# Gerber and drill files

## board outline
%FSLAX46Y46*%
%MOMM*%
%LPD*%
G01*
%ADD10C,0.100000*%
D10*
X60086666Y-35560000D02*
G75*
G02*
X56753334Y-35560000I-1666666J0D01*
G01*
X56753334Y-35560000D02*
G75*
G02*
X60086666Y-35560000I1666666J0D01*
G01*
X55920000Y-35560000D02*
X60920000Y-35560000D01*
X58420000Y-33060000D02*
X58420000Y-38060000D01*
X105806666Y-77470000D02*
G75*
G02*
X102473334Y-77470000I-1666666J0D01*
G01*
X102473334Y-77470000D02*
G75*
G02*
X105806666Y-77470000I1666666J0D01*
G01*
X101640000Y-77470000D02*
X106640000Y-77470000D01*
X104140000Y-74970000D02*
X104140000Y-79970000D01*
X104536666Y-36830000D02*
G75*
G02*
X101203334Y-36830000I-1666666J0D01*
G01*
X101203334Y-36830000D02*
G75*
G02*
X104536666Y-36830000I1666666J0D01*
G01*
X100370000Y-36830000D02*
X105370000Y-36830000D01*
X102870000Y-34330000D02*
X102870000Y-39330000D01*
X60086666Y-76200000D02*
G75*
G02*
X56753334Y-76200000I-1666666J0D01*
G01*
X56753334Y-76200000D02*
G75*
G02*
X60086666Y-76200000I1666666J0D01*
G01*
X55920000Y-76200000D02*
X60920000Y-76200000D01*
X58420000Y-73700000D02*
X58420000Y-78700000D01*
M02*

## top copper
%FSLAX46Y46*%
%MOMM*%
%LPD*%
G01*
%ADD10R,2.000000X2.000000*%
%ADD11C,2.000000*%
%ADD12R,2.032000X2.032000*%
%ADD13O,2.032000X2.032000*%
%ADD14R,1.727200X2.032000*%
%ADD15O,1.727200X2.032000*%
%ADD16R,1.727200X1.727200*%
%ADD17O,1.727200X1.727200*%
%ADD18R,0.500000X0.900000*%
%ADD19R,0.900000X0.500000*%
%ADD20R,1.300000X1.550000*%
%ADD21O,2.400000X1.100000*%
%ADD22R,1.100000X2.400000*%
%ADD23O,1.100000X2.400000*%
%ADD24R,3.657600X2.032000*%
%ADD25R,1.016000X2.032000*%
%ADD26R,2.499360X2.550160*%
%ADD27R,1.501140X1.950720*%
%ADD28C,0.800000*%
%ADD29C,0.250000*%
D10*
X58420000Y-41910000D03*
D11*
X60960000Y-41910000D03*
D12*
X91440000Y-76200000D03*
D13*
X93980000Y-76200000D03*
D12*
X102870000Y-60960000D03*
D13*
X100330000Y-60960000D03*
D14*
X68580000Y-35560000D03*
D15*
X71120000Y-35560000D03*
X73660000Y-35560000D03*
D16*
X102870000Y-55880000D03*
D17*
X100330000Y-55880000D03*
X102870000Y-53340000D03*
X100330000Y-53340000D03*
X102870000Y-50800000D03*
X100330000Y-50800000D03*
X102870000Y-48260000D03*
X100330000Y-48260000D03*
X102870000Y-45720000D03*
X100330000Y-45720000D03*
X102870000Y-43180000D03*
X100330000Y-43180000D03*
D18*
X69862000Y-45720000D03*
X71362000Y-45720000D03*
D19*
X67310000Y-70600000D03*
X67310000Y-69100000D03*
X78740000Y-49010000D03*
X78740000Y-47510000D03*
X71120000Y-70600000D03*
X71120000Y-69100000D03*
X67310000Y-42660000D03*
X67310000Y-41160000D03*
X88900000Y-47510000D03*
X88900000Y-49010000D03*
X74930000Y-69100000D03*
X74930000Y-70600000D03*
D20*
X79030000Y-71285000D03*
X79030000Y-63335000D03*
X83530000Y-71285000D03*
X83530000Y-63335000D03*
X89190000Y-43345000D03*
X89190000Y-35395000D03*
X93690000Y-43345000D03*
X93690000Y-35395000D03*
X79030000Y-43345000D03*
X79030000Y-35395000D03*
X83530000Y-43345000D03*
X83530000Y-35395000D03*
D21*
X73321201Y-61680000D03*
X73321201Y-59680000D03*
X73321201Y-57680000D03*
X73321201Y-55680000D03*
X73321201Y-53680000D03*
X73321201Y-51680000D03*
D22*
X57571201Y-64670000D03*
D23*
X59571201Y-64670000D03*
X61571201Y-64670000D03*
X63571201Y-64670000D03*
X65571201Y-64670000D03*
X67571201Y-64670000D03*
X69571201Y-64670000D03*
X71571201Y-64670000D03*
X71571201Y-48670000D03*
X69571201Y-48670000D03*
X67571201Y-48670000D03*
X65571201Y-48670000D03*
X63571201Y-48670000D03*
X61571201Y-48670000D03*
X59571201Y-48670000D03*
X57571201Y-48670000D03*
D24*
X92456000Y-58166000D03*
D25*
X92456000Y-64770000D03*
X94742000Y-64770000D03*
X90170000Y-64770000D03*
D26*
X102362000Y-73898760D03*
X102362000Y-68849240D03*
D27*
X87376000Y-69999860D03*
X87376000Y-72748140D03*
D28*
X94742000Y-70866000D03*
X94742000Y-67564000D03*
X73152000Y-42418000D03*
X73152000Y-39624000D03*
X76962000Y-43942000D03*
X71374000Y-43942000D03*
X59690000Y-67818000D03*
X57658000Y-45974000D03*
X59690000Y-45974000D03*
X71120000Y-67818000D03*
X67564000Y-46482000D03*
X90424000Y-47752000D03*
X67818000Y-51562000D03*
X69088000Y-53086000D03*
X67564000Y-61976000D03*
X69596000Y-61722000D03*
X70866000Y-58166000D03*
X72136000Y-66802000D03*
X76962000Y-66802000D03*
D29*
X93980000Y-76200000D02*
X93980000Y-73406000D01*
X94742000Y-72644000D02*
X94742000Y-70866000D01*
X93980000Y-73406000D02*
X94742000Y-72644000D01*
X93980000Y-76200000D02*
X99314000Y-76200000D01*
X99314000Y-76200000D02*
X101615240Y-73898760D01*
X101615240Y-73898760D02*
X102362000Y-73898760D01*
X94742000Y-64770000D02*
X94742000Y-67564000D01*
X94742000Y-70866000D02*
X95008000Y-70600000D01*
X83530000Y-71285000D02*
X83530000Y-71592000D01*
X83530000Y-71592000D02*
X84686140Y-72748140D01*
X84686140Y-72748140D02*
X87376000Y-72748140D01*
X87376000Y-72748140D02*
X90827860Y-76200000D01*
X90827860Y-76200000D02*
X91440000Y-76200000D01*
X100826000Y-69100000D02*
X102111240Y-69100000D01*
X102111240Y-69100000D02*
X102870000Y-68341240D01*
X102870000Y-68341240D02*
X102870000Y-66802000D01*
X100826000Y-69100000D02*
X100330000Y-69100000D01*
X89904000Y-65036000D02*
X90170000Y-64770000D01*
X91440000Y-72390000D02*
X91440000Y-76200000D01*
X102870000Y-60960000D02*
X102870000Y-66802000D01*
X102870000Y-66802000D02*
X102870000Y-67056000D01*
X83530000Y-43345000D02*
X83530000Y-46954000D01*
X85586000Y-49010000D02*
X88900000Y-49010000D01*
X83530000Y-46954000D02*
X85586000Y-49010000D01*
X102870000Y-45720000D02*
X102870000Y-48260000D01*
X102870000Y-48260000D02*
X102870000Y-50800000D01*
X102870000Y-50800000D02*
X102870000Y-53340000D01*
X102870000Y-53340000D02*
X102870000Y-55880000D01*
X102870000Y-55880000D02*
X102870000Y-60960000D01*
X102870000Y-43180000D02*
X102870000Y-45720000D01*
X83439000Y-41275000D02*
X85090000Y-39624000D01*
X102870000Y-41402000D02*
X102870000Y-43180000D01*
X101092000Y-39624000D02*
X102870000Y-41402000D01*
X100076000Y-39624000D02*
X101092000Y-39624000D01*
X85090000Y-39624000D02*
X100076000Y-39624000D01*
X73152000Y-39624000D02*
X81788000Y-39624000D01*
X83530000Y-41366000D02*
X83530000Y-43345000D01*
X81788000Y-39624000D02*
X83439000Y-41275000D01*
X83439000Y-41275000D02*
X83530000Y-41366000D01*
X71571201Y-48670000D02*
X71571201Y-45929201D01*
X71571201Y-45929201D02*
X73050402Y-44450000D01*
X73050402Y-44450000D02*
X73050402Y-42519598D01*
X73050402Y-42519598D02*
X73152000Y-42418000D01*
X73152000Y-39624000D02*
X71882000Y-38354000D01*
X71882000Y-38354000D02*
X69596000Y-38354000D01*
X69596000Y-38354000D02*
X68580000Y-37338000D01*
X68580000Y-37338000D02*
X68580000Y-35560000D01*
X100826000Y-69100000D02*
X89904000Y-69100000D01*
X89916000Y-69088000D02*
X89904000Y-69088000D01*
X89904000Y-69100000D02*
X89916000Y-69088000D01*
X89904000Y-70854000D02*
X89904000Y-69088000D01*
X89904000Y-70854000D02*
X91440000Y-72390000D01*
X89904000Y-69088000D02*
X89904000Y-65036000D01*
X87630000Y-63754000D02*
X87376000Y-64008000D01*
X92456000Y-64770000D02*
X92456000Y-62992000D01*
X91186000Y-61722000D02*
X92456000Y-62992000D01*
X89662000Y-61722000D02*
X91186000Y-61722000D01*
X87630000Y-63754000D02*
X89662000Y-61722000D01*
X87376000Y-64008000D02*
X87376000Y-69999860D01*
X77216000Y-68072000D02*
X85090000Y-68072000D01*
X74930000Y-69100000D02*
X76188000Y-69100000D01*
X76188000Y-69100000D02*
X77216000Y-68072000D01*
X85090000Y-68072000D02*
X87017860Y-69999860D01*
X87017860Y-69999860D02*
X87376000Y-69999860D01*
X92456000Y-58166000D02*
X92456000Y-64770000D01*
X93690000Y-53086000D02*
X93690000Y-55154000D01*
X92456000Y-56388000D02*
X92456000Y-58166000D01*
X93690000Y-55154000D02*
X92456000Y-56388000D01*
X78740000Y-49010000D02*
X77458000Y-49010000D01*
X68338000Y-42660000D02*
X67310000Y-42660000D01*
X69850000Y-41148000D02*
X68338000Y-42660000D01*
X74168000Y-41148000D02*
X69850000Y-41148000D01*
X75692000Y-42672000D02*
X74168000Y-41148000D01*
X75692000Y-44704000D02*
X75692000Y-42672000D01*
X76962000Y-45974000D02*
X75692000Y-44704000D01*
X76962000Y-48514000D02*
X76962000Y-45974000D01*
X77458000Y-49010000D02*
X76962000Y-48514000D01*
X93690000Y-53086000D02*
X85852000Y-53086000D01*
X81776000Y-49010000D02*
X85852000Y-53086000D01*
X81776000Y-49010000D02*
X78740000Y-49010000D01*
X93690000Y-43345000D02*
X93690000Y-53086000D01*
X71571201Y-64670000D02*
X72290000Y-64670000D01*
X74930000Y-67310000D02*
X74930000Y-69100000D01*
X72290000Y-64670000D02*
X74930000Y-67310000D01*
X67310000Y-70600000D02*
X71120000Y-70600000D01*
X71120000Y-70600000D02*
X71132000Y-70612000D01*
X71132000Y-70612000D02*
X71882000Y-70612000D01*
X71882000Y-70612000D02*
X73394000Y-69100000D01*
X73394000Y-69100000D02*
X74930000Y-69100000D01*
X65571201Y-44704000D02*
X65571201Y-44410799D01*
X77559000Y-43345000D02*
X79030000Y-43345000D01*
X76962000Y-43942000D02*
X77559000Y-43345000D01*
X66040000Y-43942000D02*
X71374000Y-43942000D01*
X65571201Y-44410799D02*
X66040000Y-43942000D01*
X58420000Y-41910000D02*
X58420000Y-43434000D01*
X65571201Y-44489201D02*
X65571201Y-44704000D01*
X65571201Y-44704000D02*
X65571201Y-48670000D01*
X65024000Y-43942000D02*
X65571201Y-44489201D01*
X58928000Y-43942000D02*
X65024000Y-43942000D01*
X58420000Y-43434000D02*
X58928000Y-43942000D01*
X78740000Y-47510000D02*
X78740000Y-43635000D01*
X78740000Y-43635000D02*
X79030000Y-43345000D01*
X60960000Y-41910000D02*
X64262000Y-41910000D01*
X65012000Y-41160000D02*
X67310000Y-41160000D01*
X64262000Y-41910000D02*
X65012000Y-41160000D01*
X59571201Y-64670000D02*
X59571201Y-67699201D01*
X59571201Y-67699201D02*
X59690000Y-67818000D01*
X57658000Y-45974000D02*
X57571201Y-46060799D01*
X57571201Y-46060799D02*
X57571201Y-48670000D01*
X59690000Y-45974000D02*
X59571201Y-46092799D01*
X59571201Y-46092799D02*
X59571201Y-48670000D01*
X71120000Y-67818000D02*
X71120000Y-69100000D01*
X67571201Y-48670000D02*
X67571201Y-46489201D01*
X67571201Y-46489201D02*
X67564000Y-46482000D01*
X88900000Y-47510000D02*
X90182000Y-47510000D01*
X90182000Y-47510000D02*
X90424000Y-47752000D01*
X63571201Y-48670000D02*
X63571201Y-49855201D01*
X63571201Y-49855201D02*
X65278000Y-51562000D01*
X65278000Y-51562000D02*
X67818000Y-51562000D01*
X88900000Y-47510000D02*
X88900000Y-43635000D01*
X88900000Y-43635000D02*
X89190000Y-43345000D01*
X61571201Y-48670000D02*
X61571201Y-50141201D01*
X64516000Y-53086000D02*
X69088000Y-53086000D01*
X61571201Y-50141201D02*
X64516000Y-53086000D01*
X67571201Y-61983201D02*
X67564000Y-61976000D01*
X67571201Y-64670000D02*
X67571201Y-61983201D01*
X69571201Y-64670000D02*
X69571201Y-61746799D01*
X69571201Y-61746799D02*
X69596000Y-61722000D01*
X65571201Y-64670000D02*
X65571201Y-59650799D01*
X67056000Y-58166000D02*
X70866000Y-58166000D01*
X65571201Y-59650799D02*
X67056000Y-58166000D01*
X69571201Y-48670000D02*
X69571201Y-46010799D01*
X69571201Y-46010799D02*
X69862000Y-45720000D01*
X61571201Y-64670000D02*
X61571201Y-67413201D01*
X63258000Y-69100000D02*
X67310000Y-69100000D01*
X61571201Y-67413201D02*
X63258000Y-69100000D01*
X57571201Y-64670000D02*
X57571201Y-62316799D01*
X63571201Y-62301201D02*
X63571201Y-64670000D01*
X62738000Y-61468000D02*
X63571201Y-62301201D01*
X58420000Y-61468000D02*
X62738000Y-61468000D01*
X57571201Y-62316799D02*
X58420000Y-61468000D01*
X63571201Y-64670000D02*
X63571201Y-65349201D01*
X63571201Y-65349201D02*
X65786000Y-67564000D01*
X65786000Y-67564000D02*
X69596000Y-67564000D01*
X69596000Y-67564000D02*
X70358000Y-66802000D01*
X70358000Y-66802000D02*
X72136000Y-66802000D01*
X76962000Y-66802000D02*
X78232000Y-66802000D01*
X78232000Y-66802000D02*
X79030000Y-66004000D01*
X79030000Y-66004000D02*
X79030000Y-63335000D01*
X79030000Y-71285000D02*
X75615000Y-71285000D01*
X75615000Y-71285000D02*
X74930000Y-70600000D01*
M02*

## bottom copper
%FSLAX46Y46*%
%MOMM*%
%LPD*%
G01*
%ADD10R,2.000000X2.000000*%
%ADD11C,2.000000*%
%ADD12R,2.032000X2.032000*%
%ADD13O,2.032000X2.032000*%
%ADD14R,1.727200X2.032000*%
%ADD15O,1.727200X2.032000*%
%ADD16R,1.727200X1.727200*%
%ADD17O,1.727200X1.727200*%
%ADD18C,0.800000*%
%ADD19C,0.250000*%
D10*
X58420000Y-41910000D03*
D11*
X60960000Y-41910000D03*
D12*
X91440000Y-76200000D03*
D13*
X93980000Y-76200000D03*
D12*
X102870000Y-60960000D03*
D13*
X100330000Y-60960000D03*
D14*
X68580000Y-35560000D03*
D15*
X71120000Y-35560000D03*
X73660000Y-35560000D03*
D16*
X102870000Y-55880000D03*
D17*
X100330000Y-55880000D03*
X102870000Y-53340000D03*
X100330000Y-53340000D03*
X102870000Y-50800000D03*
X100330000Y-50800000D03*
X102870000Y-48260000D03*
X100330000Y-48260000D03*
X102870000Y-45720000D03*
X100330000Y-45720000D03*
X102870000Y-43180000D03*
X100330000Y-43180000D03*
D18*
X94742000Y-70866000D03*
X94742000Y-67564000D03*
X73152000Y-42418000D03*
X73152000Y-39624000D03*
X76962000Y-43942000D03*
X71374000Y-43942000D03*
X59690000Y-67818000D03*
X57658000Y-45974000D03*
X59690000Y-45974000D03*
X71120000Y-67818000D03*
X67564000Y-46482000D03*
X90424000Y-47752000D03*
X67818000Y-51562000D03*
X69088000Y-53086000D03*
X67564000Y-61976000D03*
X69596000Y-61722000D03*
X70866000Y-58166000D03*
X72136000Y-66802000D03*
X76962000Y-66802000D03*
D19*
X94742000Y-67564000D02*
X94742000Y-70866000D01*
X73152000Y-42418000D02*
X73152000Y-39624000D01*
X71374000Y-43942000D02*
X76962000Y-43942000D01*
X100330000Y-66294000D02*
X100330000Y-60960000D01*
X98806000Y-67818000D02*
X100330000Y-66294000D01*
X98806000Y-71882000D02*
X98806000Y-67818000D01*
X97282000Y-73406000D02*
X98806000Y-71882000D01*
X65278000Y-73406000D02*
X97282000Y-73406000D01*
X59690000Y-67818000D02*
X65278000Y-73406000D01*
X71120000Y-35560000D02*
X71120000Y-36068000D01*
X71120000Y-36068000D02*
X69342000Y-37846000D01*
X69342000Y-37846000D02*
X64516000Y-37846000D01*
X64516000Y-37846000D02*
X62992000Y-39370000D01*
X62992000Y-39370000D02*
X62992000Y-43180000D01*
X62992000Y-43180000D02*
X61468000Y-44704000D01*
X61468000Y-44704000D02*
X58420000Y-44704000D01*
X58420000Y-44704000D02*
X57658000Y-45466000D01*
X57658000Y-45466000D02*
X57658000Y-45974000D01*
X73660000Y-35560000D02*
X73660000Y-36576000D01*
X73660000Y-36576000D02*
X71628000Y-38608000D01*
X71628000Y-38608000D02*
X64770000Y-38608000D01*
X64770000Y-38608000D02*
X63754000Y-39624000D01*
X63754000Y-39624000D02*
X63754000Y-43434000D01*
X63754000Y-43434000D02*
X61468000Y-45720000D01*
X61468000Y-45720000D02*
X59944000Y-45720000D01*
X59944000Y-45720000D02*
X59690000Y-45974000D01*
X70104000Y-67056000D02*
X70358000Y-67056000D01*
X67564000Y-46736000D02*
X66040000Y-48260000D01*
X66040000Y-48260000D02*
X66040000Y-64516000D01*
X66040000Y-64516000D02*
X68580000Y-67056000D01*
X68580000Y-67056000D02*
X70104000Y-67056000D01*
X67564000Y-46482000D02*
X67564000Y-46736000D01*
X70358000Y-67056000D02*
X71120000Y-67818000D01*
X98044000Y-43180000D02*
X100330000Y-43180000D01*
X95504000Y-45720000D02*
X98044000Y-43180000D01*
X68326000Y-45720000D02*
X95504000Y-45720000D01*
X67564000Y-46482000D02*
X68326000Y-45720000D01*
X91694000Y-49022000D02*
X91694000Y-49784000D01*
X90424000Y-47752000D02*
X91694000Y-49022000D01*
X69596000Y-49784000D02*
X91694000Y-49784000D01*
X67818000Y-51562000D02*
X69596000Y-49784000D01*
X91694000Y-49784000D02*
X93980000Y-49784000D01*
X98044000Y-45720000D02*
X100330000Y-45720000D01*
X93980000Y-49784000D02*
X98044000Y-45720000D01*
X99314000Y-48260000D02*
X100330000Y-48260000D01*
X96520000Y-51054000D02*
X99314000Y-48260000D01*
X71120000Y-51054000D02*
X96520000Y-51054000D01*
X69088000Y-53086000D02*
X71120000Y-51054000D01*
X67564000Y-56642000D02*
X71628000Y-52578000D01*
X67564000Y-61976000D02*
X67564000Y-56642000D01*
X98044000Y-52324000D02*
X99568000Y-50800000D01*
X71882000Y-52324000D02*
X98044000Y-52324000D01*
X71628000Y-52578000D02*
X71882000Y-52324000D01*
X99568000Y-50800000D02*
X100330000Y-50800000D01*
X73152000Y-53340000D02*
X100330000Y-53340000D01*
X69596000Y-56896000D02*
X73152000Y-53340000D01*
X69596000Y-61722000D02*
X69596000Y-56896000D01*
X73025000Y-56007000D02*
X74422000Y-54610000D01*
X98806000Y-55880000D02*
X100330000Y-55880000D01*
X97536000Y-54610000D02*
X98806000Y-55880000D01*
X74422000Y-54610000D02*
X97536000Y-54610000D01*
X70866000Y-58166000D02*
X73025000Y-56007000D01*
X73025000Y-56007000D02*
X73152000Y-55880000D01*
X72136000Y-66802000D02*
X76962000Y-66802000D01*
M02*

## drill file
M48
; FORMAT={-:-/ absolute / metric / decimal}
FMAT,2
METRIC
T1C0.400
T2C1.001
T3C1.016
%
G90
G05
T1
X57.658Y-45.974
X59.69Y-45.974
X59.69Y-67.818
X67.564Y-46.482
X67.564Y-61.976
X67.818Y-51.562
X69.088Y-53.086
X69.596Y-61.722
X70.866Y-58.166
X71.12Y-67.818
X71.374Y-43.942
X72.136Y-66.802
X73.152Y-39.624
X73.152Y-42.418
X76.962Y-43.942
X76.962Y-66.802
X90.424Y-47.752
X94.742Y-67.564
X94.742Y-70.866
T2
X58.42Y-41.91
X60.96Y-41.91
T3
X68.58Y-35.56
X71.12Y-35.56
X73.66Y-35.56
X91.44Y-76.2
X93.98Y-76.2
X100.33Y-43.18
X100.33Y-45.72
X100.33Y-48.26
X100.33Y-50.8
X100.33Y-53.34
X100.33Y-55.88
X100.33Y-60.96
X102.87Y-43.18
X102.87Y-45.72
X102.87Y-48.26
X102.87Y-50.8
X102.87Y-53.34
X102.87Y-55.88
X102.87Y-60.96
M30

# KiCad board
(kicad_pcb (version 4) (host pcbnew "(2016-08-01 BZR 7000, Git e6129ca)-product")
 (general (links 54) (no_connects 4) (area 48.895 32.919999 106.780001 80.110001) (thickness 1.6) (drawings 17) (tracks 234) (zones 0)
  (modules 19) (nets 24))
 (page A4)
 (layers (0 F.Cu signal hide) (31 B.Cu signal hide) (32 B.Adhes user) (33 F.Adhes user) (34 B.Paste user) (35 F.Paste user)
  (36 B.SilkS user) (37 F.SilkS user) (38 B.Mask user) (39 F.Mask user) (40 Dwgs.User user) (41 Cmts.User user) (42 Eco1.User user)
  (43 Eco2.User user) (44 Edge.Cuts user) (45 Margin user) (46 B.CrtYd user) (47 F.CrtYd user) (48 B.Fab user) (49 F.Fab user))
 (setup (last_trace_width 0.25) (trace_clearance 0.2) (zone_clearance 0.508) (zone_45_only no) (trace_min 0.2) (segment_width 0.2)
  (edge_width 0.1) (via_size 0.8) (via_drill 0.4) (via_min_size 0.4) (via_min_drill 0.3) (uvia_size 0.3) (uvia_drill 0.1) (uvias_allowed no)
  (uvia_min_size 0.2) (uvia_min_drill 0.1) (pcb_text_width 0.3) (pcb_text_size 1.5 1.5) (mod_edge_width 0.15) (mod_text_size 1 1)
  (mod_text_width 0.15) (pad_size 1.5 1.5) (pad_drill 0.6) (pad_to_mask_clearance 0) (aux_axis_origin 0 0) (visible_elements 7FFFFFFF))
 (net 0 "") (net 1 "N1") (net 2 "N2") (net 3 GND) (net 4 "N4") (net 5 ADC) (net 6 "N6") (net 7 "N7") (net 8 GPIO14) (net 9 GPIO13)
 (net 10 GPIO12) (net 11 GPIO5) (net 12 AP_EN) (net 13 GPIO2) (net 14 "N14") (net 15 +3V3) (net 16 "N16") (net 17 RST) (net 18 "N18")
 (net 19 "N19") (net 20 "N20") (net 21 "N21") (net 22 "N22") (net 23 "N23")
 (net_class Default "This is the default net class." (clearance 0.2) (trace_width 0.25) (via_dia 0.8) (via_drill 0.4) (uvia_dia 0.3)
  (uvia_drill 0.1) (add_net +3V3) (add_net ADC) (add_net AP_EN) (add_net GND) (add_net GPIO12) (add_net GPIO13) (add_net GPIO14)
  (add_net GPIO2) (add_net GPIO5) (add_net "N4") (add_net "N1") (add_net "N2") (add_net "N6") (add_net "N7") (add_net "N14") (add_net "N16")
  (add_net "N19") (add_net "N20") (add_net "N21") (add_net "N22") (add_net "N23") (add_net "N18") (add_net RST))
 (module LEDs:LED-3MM (layer F.Cu) (at 58.42 41.91)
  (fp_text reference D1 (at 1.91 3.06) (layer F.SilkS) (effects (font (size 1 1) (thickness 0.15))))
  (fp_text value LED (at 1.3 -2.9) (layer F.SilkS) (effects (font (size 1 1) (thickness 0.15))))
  (pad 1 thru_hole rect (at 0 0 90) (size 2 2) (drill 1.00076) (layers *.Cu *.Mask F.SilkS) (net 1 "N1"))
  (pad 2 thru_hole circle (at 2.54 0) (size 2 2) (drill 1.00076) (layers *.Cu *.Mask F.SilkS) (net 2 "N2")))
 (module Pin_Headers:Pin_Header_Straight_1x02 (layer F.Cu) (at 91.44 76.2 90)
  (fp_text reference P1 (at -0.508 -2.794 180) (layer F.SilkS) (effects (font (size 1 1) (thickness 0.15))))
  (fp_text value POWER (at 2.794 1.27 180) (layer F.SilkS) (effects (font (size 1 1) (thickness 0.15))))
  (pad 1 thru_hole rect (at 0 0 90) (size 2.032 2.032) (drill 1.016) (layers *.Cu *.Mask F.SilkS) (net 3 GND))
  (pad 2 thru_hole oval (at 0 2.54 90) (size 2.032 2.032) (drill 1.016) (layers *.Cu *.Mask F.SilkS) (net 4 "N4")))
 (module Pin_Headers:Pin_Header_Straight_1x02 (layer F.Cu) (at 102.87 60.96 270)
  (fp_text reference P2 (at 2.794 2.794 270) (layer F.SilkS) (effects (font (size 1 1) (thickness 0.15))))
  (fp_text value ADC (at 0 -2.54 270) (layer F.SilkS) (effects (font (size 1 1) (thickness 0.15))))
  (pad 1 thru_hole rect (at 0 0 270) (size 2.032 2.032) (drill 1.016) (layers *.Cu *.Mask F.SilkS) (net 3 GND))
  (pad 2 thru_hole oval (at 0 2.54 270) (size 2.032 2.032) (drill 1.016) (layers *.Cu *.Mask F.SilkS) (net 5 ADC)))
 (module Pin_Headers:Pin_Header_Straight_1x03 (layer F.Cu) (at 68.58 35.56 90)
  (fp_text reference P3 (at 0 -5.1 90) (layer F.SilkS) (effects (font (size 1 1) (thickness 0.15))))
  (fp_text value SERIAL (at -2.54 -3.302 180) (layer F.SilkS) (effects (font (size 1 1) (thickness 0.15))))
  (pad 1 thru_hole rect (at 0 0 90) (size 2.032 1.7272) (drill 1.016) (layers *.Cu *.Mask F.SilkS) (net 3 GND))
  (pad 2 thru_hole oval (at 0 2.54 90) (size 2.032 1.7272) (drill 1.016) (layers *.Cu *.Mask F.SilkS) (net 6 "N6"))
  (pad 3 thru_hole oval (at 0 5.08 90) (size 2.032 1.7272) (drill 1.016) (layers *.Cu *.Mask F.SilkS) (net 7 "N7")))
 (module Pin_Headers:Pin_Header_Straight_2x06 (layer F.Cu) (at 102.87 55.88 180)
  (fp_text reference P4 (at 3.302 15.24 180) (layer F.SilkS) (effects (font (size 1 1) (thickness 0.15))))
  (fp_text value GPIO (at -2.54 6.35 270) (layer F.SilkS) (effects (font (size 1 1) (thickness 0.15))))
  (pad 1 thru_hole rect (at 0 0 180) (size 1.7272 1.7272) (drill 1.016) (layers *.Cu *.Mask F.SilkS) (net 3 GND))
  (pad 2 thru_hole oval (at 2.54 0 180) (size 1.7272 1.7272) (drill 1.016) (layers *.Cu *.Mask F.SilkS) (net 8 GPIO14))
  (pad 3 thru_hole oval (at 0 2.54 180) (size 1.7272 1.7272) (drill 1.016) (layers *.Cu *.Mask F.SilkS) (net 3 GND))
  (pad 4 thru_hole oval (at 2.54 2.54 180) (size 1.7272 1.7272) (drill 1.016) (layers *.Cu *.Mask F.SilkS) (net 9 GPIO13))
  (pad 5 thru_hole oval (at 0 5.08 180) (size 1.7272 1.7272) (drill 1.016) (layers *.Cu *.Mask F.SilkS) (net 3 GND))
  (pad 6 thru_hole oval (at 2.54 5.08 180) (size 1.7272 1.7272) (drill 1.016) (layers *.Cu *.Mask F.SilkS) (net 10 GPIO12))
  (pad 7 thru_hole oval (at 0 7.62 180) (size 1.7272 1.7272) (drill 1.016) (layers *.Cu *.Mask F.SilkS) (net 3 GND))
  (pad 8 thru_hole oval (at 2.54 7.62 180) (size 1.7272 1.7272) (drill 1.016) (layers *.Cu *.Mask F.SilkS) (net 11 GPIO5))
  (pad 9 thru_hole oval (at 0 10.16 180) (size 1.7272 1.7272) (drill 1.016) (layers *.Cu *.Mask F.SilkS) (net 3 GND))
  (pad 10 thru_hole oval (at 2.54 10.16 180) (size 1.7272 1.7272) (drill 1.016) (layers *.Cu *.Mask F.SilkS) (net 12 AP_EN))
  (pad 11 thru_hole oval (at 0 12.7 180) (size 1.7272 1.7272) (drill 1.016) (layers *.Cu *.Mask F.SilkS) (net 3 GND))
  (pad 12 thru_hole oval (at 2.54 12.7 180) (size 1.7272 1.7272) (drill 1.016) (layers *.Cu *.Mask F.SilkS) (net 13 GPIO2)))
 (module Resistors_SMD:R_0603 (layer F.Cu) (at 70.612 45.72)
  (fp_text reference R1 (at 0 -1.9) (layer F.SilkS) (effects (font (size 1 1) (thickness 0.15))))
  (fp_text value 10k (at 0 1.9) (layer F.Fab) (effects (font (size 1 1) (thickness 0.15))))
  (pad 1 smd rect (at -0.75 0) (size 0.5 0.9) (layers F.Cu F.Paste F.Mask) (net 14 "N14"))
  (pad 2 smd rect (at 0.75 0) (size 0.5 0.9) (layers F.Cu F.Paste F.Mask) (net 3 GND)))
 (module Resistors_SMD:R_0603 (layer F.Cu) (at 67.31 69.85 90)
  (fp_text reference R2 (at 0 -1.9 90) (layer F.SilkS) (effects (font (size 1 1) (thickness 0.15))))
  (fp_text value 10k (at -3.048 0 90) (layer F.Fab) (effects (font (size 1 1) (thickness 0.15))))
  (pad 1 smd rect (at -0.75 0 90) (size 0.5 0.9) (layers F.Cu F.Paste F.Mask) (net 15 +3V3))
  (pad 2 smd rect (at 0.75 0 90) (size 0.5 0.9) (layers F.Cu F.Paste F.Mask) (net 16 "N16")))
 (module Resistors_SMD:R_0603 (layer F.Cu) (at 78.74 48.26 90)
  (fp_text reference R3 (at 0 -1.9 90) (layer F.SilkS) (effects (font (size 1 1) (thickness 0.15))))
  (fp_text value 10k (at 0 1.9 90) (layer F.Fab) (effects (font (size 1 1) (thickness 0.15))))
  (pad 1 smd rect (at -0.75 0 90) (size 0.5 0.9) (layers F.Cu F.Paste F.Mask) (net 15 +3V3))
  (pad 2 smd rect (at 0.75 0 90) (size 0.5 0.9) (layers F.Cu F.Paste F.Mask) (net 1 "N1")))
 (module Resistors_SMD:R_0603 (layer F.Cu) (at 71.12 69.85 90)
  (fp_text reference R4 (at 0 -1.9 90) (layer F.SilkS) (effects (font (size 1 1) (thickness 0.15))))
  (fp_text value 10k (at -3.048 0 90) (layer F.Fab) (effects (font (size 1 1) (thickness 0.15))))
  (pad 1 smd rect (at -0.75 0 90) (size 0.5 0.9) (layers F.Cu F.Paste F.Mask) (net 15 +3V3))
  (pad 2 smd rect (at 0.75 0 90) (size 0.5 0.9) (layers F.Cu F.Paste F.Mask) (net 13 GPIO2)))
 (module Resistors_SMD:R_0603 (layer F.Cu) (at 67.31 41.91 90)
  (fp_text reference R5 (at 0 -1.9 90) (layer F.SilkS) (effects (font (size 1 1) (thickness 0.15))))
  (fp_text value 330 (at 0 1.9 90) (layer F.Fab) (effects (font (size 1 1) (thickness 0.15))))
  (pad 1 smd rect (at -0.75 0 90) (size 0.5 0.9) (layers F.Cu F.Paste F.Mask) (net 15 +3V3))
  (pad 2 smd rect (at 0.75 0 90) (size 0.5 0.9) (layers F.Cu F.Paste F.Mask) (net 2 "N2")))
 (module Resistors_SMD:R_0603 (layer F.Cu) (at 88.9 48.26 270)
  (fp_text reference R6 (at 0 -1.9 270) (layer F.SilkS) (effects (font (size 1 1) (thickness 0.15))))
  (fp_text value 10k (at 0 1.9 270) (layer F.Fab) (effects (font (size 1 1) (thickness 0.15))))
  (pad 1 smd rect (at -0.75 0 270) (size 0.5 0.9) (layers F.Cu F.Paste F.Mask) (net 12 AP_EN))
  (pad 2 smd rect (at 0.75 0 270) (size 0.5 0.9) (layers F.Cu F.Paste F.Mask) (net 3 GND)))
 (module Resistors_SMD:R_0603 (layer F.Cu) (at 74.93 69.85 270)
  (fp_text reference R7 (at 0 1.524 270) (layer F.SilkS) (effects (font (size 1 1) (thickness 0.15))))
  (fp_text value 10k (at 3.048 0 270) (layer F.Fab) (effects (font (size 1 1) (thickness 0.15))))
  (pad 1 smd rect (at -0.75 0 270) (size 0.5 0.9) (layers F.Cu F.Paste F.Mask) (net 15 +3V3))
  (pad 2 smd rect (at 0.75 0 270) (size 0.5 0.9) (layers F.Cu F.Paste F.Mask) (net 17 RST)))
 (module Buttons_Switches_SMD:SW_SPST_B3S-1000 (layer F.Cu) (at 81.28 67.31 90)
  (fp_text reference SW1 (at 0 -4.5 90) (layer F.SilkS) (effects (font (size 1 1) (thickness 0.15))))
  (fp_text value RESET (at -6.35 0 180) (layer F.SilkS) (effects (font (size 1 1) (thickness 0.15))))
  (pad 1 smd rect (at -3.975 -2.25 90) (size 1.55 1.3) (layers F.Cu F.Paste F.Mask) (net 17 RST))
  (pad 1 smd rect (at 3.975 -2.25 90) (size 1.55 1.3) (layers F.Cu F.Paste F.Mask) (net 17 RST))
  (pad 2 smd rect (at -3.975 2.25 90) (size 1.55 1.3) (layers F.Cu F.Paste F.Mask) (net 3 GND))
  (pad 2 smd rect (at 3.975 2.25 90) (size 1.55 1.3) (layers F.Cu F.Paste F.Mask) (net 3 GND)))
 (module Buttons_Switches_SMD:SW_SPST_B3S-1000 (layer F.Cu) (at 91.44 39.37 90)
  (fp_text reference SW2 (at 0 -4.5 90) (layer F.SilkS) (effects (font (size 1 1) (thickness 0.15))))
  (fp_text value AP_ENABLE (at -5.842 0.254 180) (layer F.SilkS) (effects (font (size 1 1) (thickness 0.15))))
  (pad 1 smd rect (at -3.975 -2.25 90) (size 1.55 1.3) (layers F.Cu F.Paste F.Mask) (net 12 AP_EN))
  (pad 1 smd rect (at 3.975 -2.25 90) (size 1.55 1.3) (layers F.Cu F.Paste F.Mask) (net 12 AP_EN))
  (pad 2 smd rect (at -3.975 2.25 90) (size 1.55 1.3) (layers F.Cu F.Paste F.Mask) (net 15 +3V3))
  (pad 2 smd rect (at 3.975 2.25 90) (size 1.55 1.3) (layers F.Cu F.Paste F.Mask) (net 15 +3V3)))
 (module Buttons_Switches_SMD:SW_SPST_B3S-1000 (layer F.Cu) (at 81.28 39.37 90)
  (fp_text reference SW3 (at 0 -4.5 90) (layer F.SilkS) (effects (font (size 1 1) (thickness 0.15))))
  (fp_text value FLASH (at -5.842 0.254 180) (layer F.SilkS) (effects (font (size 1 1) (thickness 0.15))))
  (pad 1 smd rect (at -3.975 -2.25 90) (size 1.55 1.3) (layers F.Cu F.Paste F.Mask) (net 1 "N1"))
  (pad 1 smd rect (at 3.975 -2.25 90) (size 1.55 1.3) (layers F.Cu F.Paste F.Mask) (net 1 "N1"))
  (pad 2 smd rect (at -3.975 2.25 90) (size 1.55 1.3) (layers F.Cu F.Paste F.Mask) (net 3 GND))
  (pad 2 smd rect (at 3.975 2.25 90) (size 1.55 1.3) (layers F.Cu F.Paste F.Mask) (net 3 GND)))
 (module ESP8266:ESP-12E (layer F.Cu) (at 57.571201 64.67 90)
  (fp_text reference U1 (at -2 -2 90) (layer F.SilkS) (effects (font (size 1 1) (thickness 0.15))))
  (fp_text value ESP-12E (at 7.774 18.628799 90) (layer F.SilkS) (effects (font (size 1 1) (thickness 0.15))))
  (pad 9 smd oval (at 2.99 15.75 180) (size 2.4 1.1) (layers F.Cu F.Paste F.Mask) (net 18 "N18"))
  (pad 10 smd oval (at 4.99 15.75 180) (size 2.4 1.1) (layers F.Cu F.Paste F.Mask) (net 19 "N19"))
  (pad 11 smd oval (at 6.99 15.75 180) (size 2.4 1.1) (layers F.Cu F.Paste F.Mask) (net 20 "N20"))
  (pad 12 smd oval (at 8.99 15.75 180) (size 2.4 1.1) (layers F.Cu F.Paste F.Mask) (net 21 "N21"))
  (pad 13 smd oval (at 10.99 15.75 180) (size 2.4 1.1) (layers F.Cu F.Paste F.Mask) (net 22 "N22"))
  (pad 14 smd oval (at 12.99 15.75 180) (size 2.4 1.1) (layers F.Cu F.Paste F.Mask) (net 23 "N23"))
  (pad 1 smd rect (at 0 0 90) (size 2.4 1.1) (layers F.Cu F.Paste F.Mask) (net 17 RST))
  (pad 2 smd oval (at 0 2 90) (size 2.4 1.1) (layers F.Cu F.Paste F.Mask) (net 5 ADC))
  (pad 3 smd oval (at 0 4 90) (size 2.4 1.1) (layers F.Cu F.Paste F.Mask) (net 16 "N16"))
  (pad 4 smd oval (at 0 6 90) (size 2.4 1.1) (layers F.Cu F.Paste F.Mask) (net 17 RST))
  (pad 5 smd oval (at 0 8 90) (size 2.4 1.1) (layers F.Cu F.Paste F.Mask) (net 8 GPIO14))
  (pad 6 smd oval (at 0 10 90) (size 2.4 1.1) (layers F.Cu F.Paste F.Mask) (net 10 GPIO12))
  (pad 7 smd oval (at 0 12 90) (size 2.4 1.1) (layers F.Cu F.Paste F.Mask) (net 9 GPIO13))
  (pad 8 smd oval (at 0 14 90) (size 2.4 1.1) (layers F.Cu F.Paste F.Mask) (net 15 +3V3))
  (pad 15 smd oval (at 16 14 90) (size 2.4 1.1) (layers F.Cu F.Paste F.Mask) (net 3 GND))
  (pad 16 smd oval (at 16 12 90) (size 2.4 1.1) (layers F.Cu F.Paste F.Mask) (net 14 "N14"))
  (pad 17 smd oval (at 16 10 90) (size 2.4 1.1) (layers F.Cu F.Paste F.Mask) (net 13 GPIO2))
  (pad 18 smd oval (at 16 8 90) (size 2.4 1.1) (layers F.Cu F.Paste F.Mask) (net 1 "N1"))
  (pad 19 smd oval (at 16 6 90) (size 2.4 1.1) (layers F.Cu F.Paste F.Mask) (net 12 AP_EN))
  (pad 20 smd oval (at 16 4 90) (size 2.4 1.1) (layers F.Cu F.Paste F.Mask) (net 11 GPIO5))
  (pad 21 smd oval (at 16 2 90) (size 2.4 1.1) (layers F.Cu F.Paste F.Mask) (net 7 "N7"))
  (pad 22 smd oval (at 16 0 90) (size 2.4 1.1) (layers F.Cu F.Paste F.Mask) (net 6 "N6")))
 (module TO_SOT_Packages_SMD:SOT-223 (layer F.Cu) (at 92.456 61.468)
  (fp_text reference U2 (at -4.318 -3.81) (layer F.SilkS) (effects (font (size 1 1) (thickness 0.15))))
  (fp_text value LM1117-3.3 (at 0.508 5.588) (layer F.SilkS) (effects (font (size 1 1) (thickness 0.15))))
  (pad 4 smd rect (at 0 -3.302) (size 3.6576 2.032) (layers F.Cu F.Paste F.Mask) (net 15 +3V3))
  (pad 2 smd rect (at 0 3.302) (size 1.016 2.032) (layers F.Cu F.Paste F.Mask) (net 15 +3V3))
  (pad 3 smd rect (at 2.286 3.302) (size 1.016 2.032) (layers F.Cu F.Paste F.Mask) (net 4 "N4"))
  (pad 1 smd rect (at -2.286 3.302) (size 1.016 2.032) (layers F.Cu F.Paste F.Mask) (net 3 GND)))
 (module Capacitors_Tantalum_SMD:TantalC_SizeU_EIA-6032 (layer F.Cu) (at 102.362 71.374 270)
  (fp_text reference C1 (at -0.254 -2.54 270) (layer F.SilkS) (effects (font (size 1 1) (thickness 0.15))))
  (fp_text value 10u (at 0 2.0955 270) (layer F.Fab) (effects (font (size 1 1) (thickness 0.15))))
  (pad 1 smd rect (at 2.52476 0 270) (size 2.55016 2.49936) (layers F.Cu F.Paste F.Mask) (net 4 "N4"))
  (pad 2 smd rect (at -2.52476 0 270) (size 2.55016 2.49936) (layers F.Cu F.Paste F.Mask) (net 3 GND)))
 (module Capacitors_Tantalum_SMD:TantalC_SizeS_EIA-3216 (layer F.Cu) (at 87.376 71.374 90)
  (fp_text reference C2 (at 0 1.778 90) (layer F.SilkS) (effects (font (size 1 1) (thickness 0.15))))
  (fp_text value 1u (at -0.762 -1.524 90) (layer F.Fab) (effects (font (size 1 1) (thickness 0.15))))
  (pad 1 smd rect (at 1.37414 0 90) (size 1.95072 1.50114) (layers F.Cu F.Paste F.Mask) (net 15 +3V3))
  (pad 2 smd rect (at -1.37414 0 90) (size 1.95072 1.50114) (layers F.Cu F.Paste F.Mask) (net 3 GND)))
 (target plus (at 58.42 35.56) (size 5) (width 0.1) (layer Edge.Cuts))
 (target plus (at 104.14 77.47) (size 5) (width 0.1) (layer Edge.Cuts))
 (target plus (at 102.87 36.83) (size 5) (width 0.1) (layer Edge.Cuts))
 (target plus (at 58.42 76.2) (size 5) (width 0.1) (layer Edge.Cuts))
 (segment (start 93.98 76.2) (end 93.98 73.406) (width 0.25) (layer F.Cu) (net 4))
 (segment (start 94.742 72.644) (end 94.742 70.866) (width 0.25) (layer F.Cu) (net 4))
 (segment (start 93.98 73.406) (end 94.742 72.644) (width 0.25) (layer F.Cu) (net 4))
 (segment (start 93.98 76.2) (end 99.314 76.2) (width 0.25) (layer F.Cu) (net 4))
 (segment (start 99.314 76.2) (end 101.61524 73.89876) (width 0.25) (layer F.Cu) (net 4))
 (segment (start 101.61524 73.89876) (end 102.362 73.89876) (width 0.25) (layer F.Cu) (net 4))
 (via (at 94.742 70.866) (size 0.8) (drill 0.4) (layers F.Cu B.Cu) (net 4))
 (segment (start 94.742 64.77) (end 94.742 67.564) (width 0.25) (layer F.Cu) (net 4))
 (segment (start 94.742 67.564) (end 94.742 70.866) (width 0.25) (layer B.Cu) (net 4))
 (via (at 94.742 67.564) (size 0.8) (drill 0.4) (layers F.Cu B.Cu) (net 4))
 (segment (start 94.742 70.866) (end 95.008 70.6) (width 0.25) (layer F.Cu) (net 4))
 (segment (start 83.53 71.285) (end 83.53 71.592) (width 0.25) (layer F.Cu) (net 3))
 (segment (start 83.53 71.592) (end 84.68614 72.74814) (width 0.25) (layer F.Cu) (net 3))
 (segment (start 84.68614 72.74814) (end 87.376 72.74814) (width 0.25) (layer F.Cu) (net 3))
 (segment (start 87.376 72.74814) (end 90.82786 76.2) (width 0.25) (layer F.Cu) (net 3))
 (segment (start 90.82786 76.2) (end 91.44 76.2) (width 0.25) (layer F.Cu) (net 3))
 (segment (start 100.826 69.1) (end 102.11124 69.1) (width 0.25) (layer F.Cu) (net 3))
 (segment (start 102.11124 69.1) (end 102.87 68.34124) (width 0.25) (layer F.Cu) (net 3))
 (segment (start 102.87 68.34124) (end 102.87 66.802) (width 0.25) (layer F.Cu) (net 3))
 (segment (start 100.826 69.1) (end 100.33 69.1) (width 0.25) (layer F.Cu) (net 3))
 (segment (start 89.904 65.036) (end 90.17 64.77) (width 0.25) (layer F.Cu) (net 3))
 (segment (start 91.44 72.39) (end 91.44 76.2) (width 0.25) (layer F.Cu) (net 3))
 (segment (start 102.87 60.96) (end 102.87 66.802) (width 0.25) (layer F.Cu) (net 3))
 (segment (start 102.87 66.802) (end 102.87 67.056) (width 0.25) (layer F.Cu) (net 3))
 (segment (start 83.53 43.345) (end 83.53 46.954) (width 0.25) (layer F.Cu) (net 3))
 (segment (start 85.586 49.01) (end 88.9 49.01) (width 0.25) (layer F.Cu) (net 3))
 (segment (start 83.53 46.954) (end 85.586 49.01) (width 0.25) (layer F.Cu) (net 3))
 (segment (start 102.87 45.72) (end 102.87 48.26) (width 0.25) (layer F.Cu) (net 3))
 (segment (start 102.87 48.26) (end 102.87 50.8) (width 0.25) (layer F.Cu) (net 3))
 (segment (start 102.87 50.8) (end 102.87 53.34) (width 0.25) (layer F.Cu) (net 3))
 (segment (start 102.87 53.34) (end 102.87 55.88) (width 0.25) (layer F.Cu) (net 3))
 (segment (start 102.87 55.88) (end 102.87 60.96) (width 0.25) (layer F.Cu) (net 3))
 (segment (start 102.87 43.18) (end 102.87 45.72) (width 0.25) (layer F.Cu) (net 3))
 (segment (start 83.439 41.275) (end 85.09 39.624) (width 0.25) (layer F.Cu) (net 3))
 (segment (start 102.87 41.402) (end 102.87 43.18) (width 0.25) (layer F.Cu) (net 3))
 (segment (start 101.092 39.624) (end 102.87 41.402) (width 0.25) (layer F.Cu) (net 3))
 (segment (start 100.076 39.624) (end 101.092 39.624) (width 0.25) (layer F.Cu) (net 3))
 (segment (start 85.09 39.624) (end 100.076 39.624) (width 0.25) (layer F.Cu) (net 3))
 (segment (start 73.152 39.624) (end 81.788 39.624) (width 0.25) (layer F.Cu) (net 3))
 (segment (start 83.53 41.366) (end 83.53 43.345) (width 0.25) (layer F.Cu) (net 3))
 (segment (start 81.788 39.624) (end 83.439 41.275) (width 0.25) (layer F.Cu) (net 3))
 (segment (start 83.439 41.275) (end 83.53 41.366) (width 0.25) (layer F.Cu) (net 3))
 (segment (start 71.571201 48.67) (end 71.571201 45.929201) (width 0.25) (layer F.Cu) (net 3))
 (segment (start 71.571201 45.929201) (end 73.050402 44.45) (width 0.25) (layer F.Cu) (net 3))
 (segment (start 73.050402 44.45) (end 73.050402 42.519598) (width 0.25) (layer F.Cu) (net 3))
 (segment (start 73.050402 42.519598) (end 73.152 42.418) (width 0.25) (layer F.Cu) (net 3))
 (via (at 73.152 42.418) (size 0.8) (drill 0.4) (layers F.Cu B.Cu) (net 3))
 (segment (start 73.152 42.418) (end 73.152 39.624) (width 0.25) (layer B.Cu) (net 3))
 (via (at 73.152 39.624) (size 0.8) (drill 0.4) (layers F.Cu B.Cu) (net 3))
 (segment (start 73.152 39.624) (end 71.882 38.354) (width 0.25) (layer F.Cu) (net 3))
 (segment (start 71.882 38.354) (end 69.596 38.354) (width 0.25) (layer F.Cu) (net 3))
 (segment (start 69.596 38.354) (end 68.58 37.338) (width 0.25) (layer F.Cu) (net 3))
 (segment (start 68.58 37.338) (end 68.58 35.56) (width 0.25) (layer F.Cu) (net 3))
 (segment (start 100.826 69.1) (end 89.904 69.1) (width 0.25) (layer F.Cu) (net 3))
 (segment (start 89.916 69.088) (end 89.904 69.088) (width 0.25) (layer F.Cu) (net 3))
 (segment (start 89.904 69.1) (end 89.916 69.088) (width 0.25) (layer F.Cu) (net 3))
 (segment (start 89.904 70.854) (end 89.904 69.088) (width 0.25) (layer F.Cu) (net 3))
 (segment (start 89.904 70.854) (end 91.44 72.39) (width 0.25) (layer F.Cu) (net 3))
 (segment (start 89.904 69.088) (end 89.904 65.036) (width 0.25) (layer F.Cu) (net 3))
 (segment (start 87.63 63.754) (end 87.376 64.008) (width 0.25) (layer F.Cu) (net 15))
 (segment (start 92.456 64.77) (end 92.456 62.992) (width 0.25) (layer F.Cu) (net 15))
 (segment (start 91.186 61.722) (end 92.456 62.992) (width 0.25) (layer F.Cu) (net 15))
 (segment (start 89.662 61.722) (end 91.186 61.722) (width 0.25) (layer F.Cu) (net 15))
 (segment (start 87.63 63.754) (end 89.662 61.722) (width 0.25) (layer F.Cu) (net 15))
 (segment (start 87.376 64.008) (end 87.376 69.99986) (width 0.25) (layer F.Cu) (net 15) (status 800000))
 (segment (start 77.216 68.072) (end 85.09 68.072) (width 0.25) (layer F.Cu) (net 15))
 (segment (start 74.93 69.1) (end 76.188 69.1) (width 0.25) (layer F.Cu) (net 15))
 (segment (start 76.188 69.1) (end 77.216 68.072) (width 0.25) (layer F.Cu) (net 15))
 (segment (start 85.09 68.072) (end 87.01786 69.99986) (width 0.25) (layer F.Cu) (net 15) (status 800000))
 (segment (start 87.01786 69.99986) (end 87.376 69.99986) (width 0.25) (layer F.Cu) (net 15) (status C00000))
 (segment (start 92.456 58.166) (end 92.456 64.77) (width 0.25) (layer F.Cu) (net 15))
 (segment (start 93.69 53.086) (end 93.69 55.154) (width 0.25) (layer F.Cu) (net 15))
 (segment (start 92.456 56.388) (end 92.456 58.166) (width 0.25) (layer F.Cu) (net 15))
 (segment (start 93.69 55.154) (end 92.456 56.388) (width 0.25) (layer F.Cu) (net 15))
 (segment (start 78.74 49.01) (end 77.458 49.01) (width 0.25) (layer F.Cu) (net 15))
 (segment (start 68.338 42.66) (end 67.31 42.66) (width 0.25) (layer F.Cu) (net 15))
 (segment (start 69.85 41.148) (end 68.338 42.66) (width 0.25) (layer F.Cu) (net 15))
 (segment (start 74.168 41.148) (end 69.85 41.148) (width 0.25) (layer F.Cu) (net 15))
 (segment (start 75.692 42.672) (end 74.168 41.148) (width 0.25) (layer F.Cu) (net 15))
 (segment (start 75.692 44.704) (end 75.692 42.672) (width 0.25) (layer F.Cu) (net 15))
 (segment (start 76.962 45.974) (end 75.692 44.704) (width 0.25) (layer F.Cu) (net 15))
 (segment (start 76.962 48.514) (end 76.962 45.974) (width 0.25) (layer F.Cu) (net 15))
 (segment (start 77.458 49.01) (end 76.962 48.514) (width 0.25) (layer F.Cu) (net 15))
 (segment (start 93.69 53.086) (end 85.852 53.086) (width 0.25) (layer F.Cu) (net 15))
 (segment (start 81.776 49.01) (end 85.852 53.086) (width 0.25) (layer F.Cu) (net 15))
 (segment (start 81.776 49.01) (end 78.74 49.01) (width 0.25) (layer F.Cu) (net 15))
 (segment (start 93.69 43.345) (end 93.69 53.086) (width 0.25) (layer F.Cu) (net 15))
 (segment (start 71.571201 64.67) (end 72.29 64.67) (width 0.25) (layer F.Cu) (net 15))
 (segment (start 74.93 67.31) (end 74.93 69.1) (width 0.25) (layer F.Cu) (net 15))
 (segment (start 72.29 64.67) (end 74.93 67.31) (width 0.25) (layer F.Cu) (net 15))
 (segment (start 67.31 70.6) (end 71.12 70.6) (width 0.25) (layer F.Cu) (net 15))
 (segment (start 71.12 70.6) (end 71.132 70.612) (width 0.25) (layer F.Cu) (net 15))
 (segment (start 71.132 70.612) (end 71.882 70.612) (width 0.25) (layer F.Cu) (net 15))
 (segment (start 71.882 70.612) (end 73.394 69.1) (width 0.25) (layer F.Cu) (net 15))
 (segment (start 73.394 69.1) (end 74.93 69.1) (width 0.25) (layer F.Cu) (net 15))
 (segment (start 65.571201 44.704) (end 65.571201 44.410799) (width 0.25) (layer F.Cu) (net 1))
 (segment (start 77.559 43.345) (end 79.03 43.345) (width 0.25) (layer F.Cu) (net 1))
 (segment (start 76.962 43.942) (end 77.559 43.345) (width 0.25) (layer F.Cu) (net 1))
 (via (at 76.962 43.942) (size 0.8) (drill 0.4) (layers F.Cu B.Cu) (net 1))
 (segment (start 71.374 43.942) (end 76.962 43.942) (width 0.25) (layer B.Cu) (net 1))
 (via (at 71.374 43.942) (size 0.8) (drill 0.4) (layers F.Cu B.Cu) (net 1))
 (segment (start 66.04 43.942) (end 71.374 43.942) (width 0.25) (layer F.Cu) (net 1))
 (segment (start 65.571201 44.410799) (end 66.04 43.942) (width 0.25) (layer F.Cu) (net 1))
 (segment (start 58.42 41.91) (end 58.42 43.434) (width 0.25) (layer F.Cu) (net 1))
 (segment (start 65.571201 44.489201) (end 65.571201 44.704) (width 0.25) (layer F.Cu) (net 1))
 (segment (start 65.571201 44.704) (end 65.571201 48.67) (width 0.25) (layer F.Cu) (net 1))
 (segment (start 65.024 43.942) (end 65.571201 44.489201) (width 0.25) (layer F.Cu) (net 1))
 (segment (start 58.928 43.942) (end 65.024 43.942) (width 0.25) (layer F.Cu) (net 1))
 (segment (start 58.42 43.434) (end 58.928 43.942) (width 0.25) (layer F.Cu) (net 1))
 (segment (start 78.74 47.51) (end 78.74 43.635) (width 0.25) (layer F.Cu) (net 1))
 (segment (start 78.74 43.635) (end 79.03 43.345) (width 0.25) (layer F.Cu) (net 1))
 (segment (start 60.96 41.91) (end 64.262 41.91) (width 0.25) (layer F.Cu) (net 2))
 (segment (start 65.012 41.16) (end 67.31 41.16) (width 0.25) (layer F.Cu) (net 2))
 (segment (start 64.262 41.91) (end 65.012 41.16) (width 0.25) (layer F.Cu) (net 2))
 (segment (start 59.571201 64.67) (end 59.571201 67.699201) (width 0.25) (layer F.Cu) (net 5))
 (segment (start 100.33 66.294) (end 100.33 60.96) (width 0.25) (layer B.Cu) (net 5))
 (segment (start 98.806 67.818) (end 100.33 66.294) (width 0.25) (layer B.Cu) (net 5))
 (segment (start 98.806 71.882) (end 98.806 67.818) (width 0.25) (layer B.Cu) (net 5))
 (segment (start 97.282 73.406) (end 98.806 71.882) (width 0.25) (layer B.Cu) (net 5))
 (segment (start 65.278 73.406) (end 97.282 73.406) (width 0.25) (layer B.Cu) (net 5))
 (segment (start 59.69 67.818) (end 65.278 73.406) (width 0.25) (layer B.Cu) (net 5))
 (via (at 59.69 67.818) (size 0.8) (drill 0.4) (layers F.Cu B.Cu) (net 5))
 (segment (start 59.571201 67.699201) (end 59.69 67.818) (width 0.25) (layer F.Cu) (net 5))
 (segment (start 71.12 35.56) (end 71.12 36.068) (width 0.25) (layer B.Cu) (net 6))
 (segment (start 71.12 36.068) (end 69.342 37.846) (width 0.25) (layer B.Cu) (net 6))
 (segment (start 69.342 37.846) (end 64.516 37.846) (width 0.25) (layer B.Cu) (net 6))
 (segment (start 64.516 37.846) (end 62.992 39.37) (width 0.25) (layer B.Cu) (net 6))
 (segment (start 62.992 39.37) (end 62.992 43.18) (width 0.25) (layer B.Cu) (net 6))
 (segment (start 62.992 43.18) (end 61.468 44.704) (width 0.25) (layer B.Cu) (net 6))
 (segment (start 61.468 44.704) (end 58.42 44.704) (width 0.25) (layer B.Cu) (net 6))
 (segment (start 58.42 44.704) (end 57.658 45.466) (width 0.25) (layer B.Cu) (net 6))
 (segment (start 57.658 45.466) (end 57.658 45.974) (width 0.25) (layer B.Cu) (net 6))
 (via (at 57.658 45.974) (size 0.8) (drill 0.4) (layers F.Cu B.Cu) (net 6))
 (segment (start 57.658 45.974) (end 57.571201 46.060799) (width 0.25) (layer F.Cu) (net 6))
 (segment (start 57.571201 46.060799) (end 57.571201 48.67) (width 0.25) (layer F.Cu) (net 6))
 (segment (start 73.66 35.56) (end 73.66 36.576) (width 0.25) (layer B.Cu) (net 7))
 (segment (start 73.66 36.576) (end 71.628 38.608) (width 0.25) (layer B.Cu) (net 7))
 (segment (start 71.628 38.608) (end 64.77 38.608) (width 0.25) (layer B.Cu) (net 7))
 (segment (start 64.77 38.608) (end 63.754 39.624) (width 0.25) (layer B.Cu) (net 7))
 (segment (start 63.754 39.624) (end 63.754 43.434) (width 0.25) (layer B.Cu) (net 7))
 (segment (start 63.754 43.434) (end 61.468 45.72) (width 0.25) (layer B.Cu) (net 7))
 (segment (start 61.468 45.72) (end 59.944 45.72) (width 0.25) (layer B.Cu) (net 7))
 (segment (start 59.944 45.72) (end 59.69 45.974) (width 0.25) (layer B.Cu) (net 7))
 (via (at 59.69 45.974) (size 0.8) (drill 0.4) (layers F.Cu B.Cu) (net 7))
 (segment (start 59.69 45.974) (end 59.571201 46.092799) (width 0.25) (layer F.Cu) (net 7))
 (segment (start 59.571201 46.092799) (end 59.571201 48.67) (width 0.25) (layer F.Cu) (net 7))
 (segment (start 70.104 67.056) (end 70.358 67.056) (width 0.25) (layer B.Cu) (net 13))
 (segment (start 67.564 46.736) (end 66.04 48.26) (width 0.25) (layer B.Cu) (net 13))
 (segment (start 66.04 48.26) (end 66.04 64.516) (width 0.25) (layer B.Cu) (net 13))
 (segment (start 66.04 64.516) (end 68.58 67.056) (width 0.25) (layer B.Cu) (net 13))
 (segment (start 68.58 67.056) (end 70.104 67.056) (width 0.25) (layer B.Cu) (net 13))
 (segment (start 67.564 46.482) (end 67.564 46.736) (width 0.25) (layer B.Cu) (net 13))
 (segment (start 71.12 67.818) (end 71.12 69.1) (width 0.25) (layer F.Cu) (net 13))
 (via (at 71.12 67.818) (size 0.8) (drill 0.4) (layers F.Cu B.Cu) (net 13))
 (segment (start 70.358 67.056) (end 71.12 67.818) (width 0.25) (layer B.Cu) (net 13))
 (segment (start 67.571201 48.67) (end 67.571201 46.489201) (width 0.25) (layer F.Cu) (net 13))
 (segment (start 98.044 43.18) (end 100.33 43.18) (width 0.25) (layer B.Cu) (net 13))
 (segment (start 95.504 45.72) (end 98.044 43.18) (width 0.25) (layer B.Cu) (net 13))
 (segment (start 68.326 45.72) (end 95.504 45.72) (width 0.25) (layer B.Cu) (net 13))
 (segment (start 67.564 46.482) (end 68.326 45.72) (width 0.25) (layer B.Cu) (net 13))
 (via (at 67.564 46.482) (size 0.8) (drill 0.4) (layers F.Cu B.Cu) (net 13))
 (segment (start 67.571201 46.489201) (end 67.564 46.482) (width 0.25) (layer F.Cu) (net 13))
 (segment (start 88.9 47.51) (end 90.182 47.51) (width 0.25) (layer F.Cu) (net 12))
 (segment (start 91.694 49.022) (end 91.694 49.784) (width 0.25) (layer B.Cu) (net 12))
 (segment (start 90.424 47.752) (end 91.694 49.022) (width 0.25) (layer B.Cu) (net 12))
 (via (at 90.424 47.752) (size 0.8) (drill 0.4) (layers F.Cu B.Cu) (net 12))
 (segment (start 90.182 47.51) (end 90.424 47.752) (width 0.25) (layer F.Cu) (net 12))
 (segment (start 63.571201 48.67) (end 63.571201 49.855201) (width 0.25) (layer F.Cu) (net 12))
 (segment (start 63.571201 49.855201) (end 65.278 51.562) (width 0.25) (layer F.Cu) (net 12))
 (segment (start 69.596 49.784) (end 91.694 49.784) (width 0.25) (layer B.Cu) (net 12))
 (segment (start 67.818 51.562) (end 69.596 49.784) (width 0.25) (layer B.Cu) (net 12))
 (via (at 67.818 51.562) (size 0.8) (drill 0.4) (layers F.Cu B.Cu) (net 12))
 (segment (start 65.278 51.562) (end 67.818 51.562) (width 0.25) (layer F.Cu) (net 12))
 (segment (start 91.694 49.784) (end 93.98 49.784) (width 0.25) (layer B.Cu) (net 12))
 (segment (start 98.044 45.72) (end 100.33 45.72) (width 0.25) (layer B.Cu) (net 12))
 (segment (start 93.98 49.784) (end 98.044 45.72) (width 0.25) (layer B.Cu) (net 12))
 (segment (start 88.9 47.51) (end 88.9 43.635) (width 0.25) (layer F.Cu) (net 12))
 (segment (start 88.9 43.635) (end 89.19 43.345) (width 0.25) (layer F.Cu) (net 12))
 (segment (start 61.571201 48.67) (end 61.571201 50.141201) (width 0.25) (layer F.Cu) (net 11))
 (segment (start 99.314 48.26) (end 100.33 48.26) (width 0.25) (layer B.Cu) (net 11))
 (segment (start 96.52 51.054) (end 99.314 48.26) (width 0.25) (layer B.Cu) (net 11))
 (segment (start 71.12 51.054) (end 96.52 51.054) (width 0.25) (layer B.Cu) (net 11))
 (segment (start 69.088 53.086) (end 71.12 51.054) (width 0.25) (layer B.Cu) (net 11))
 (via (at 69.088 53.086) (size 0.8) (drill 0.4) (layers F.Cu B.Cu) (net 11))
 (segment (start 64.516 53.086) (end 69.088 53.086) (width 0.25) (layer F.Cu) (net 11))
 (segment (start 61.571201 50.141201) (end 64.516 53.086) (width 0.25) (layer F.Cu) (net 11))
 (segment (start 67.564 56.642) (end 71.628 52.578) (width 0.25) (layer B.Cu) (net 10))
 (segment (start 67.571201 61.983201) (end 67.564 61.976) (width 0.25) (layer F.Cu) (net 10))
 (via (at 67.564 61.976) (size 0.8) (drill 0.4) (layers F.Cu B.Cu) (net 10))
 (segment (start 67.564 61.976) (end 67.564 56.642) (width 0.25) (layer B.Cu) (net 10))
 (segment (start 67.571201 64.67) (end 67.571201 61.983201) (width 0.25) (layer F.Cu) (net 10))
 (segment (start 98.044 52.324) (end 99.568 50.8) (width 0.25) (layer B.Cu) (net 10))
 (segment (start 71.882 52.324) (end 98.044 52.324) (width 0.25) (layer B.Cu) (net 10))
 (segment (start 71.628 52.578) (end 71.882 52.324) (width 0.25) (layer B.Cu) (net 10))
 (segment (start 99.568 50.8) (end 100.33 50.8) (width 0.25) (layer B.Cu) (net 10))
 (segment (start 69.571201 64.67) (end 69.571201 61.746799) (width 0.25) (layer F.Cu) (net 9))
 (segment (start 73.152 53.34) (end 100.33 53.34) (width 0.25) (layer B.Cu) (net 9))
 (segment (start 69.596 56.896) (end 73.152 53.34) (width 0.25) (layer B.Cu) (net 9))
 (segment (start 69.596 61.722) (end 69.596 56.896) (width 0.25) (layer B.Cu) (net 9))
 (via (at 69.596 61.722) (size 0.8) (drill 0.4) (layers F.Cu B.Cu) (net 9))
 (segment (start 69.571201 61.746799) (end 69.596 61.722) (width 0.25) (layer F.Cu) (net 9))
 (segment (start 73.025 56.007) (end 74.422 54.61) (width 0.25) (layer B.Cu) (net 8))
 (segment (start 98.806 55.88) (end 100.33 55.88) (width 0.25) (layer B.Cu) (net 8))
 (segment (start 97.536 54.61) (end 98.806 55.88) (width 0.25) (layer B.Cu) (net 8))
 (segment (start 74.422 54.61) (end 97.536 54.61) (width 0.25) (layer B.Cu) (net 8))
 (segment (start 65.571201 64.67) (end 65.571201 59.650799) (width 0.25) (layer F.Cu) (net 8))
 (segment (start 70.866 58.166) (end 73.025 56.007) (width 0.25) (layer B.Cu) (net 8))
 (segment (start 73.025 56.007) (end 73.152 55.88) (width 0.25) (layer B.Cu) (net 8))
 (via (at 70.866 58.166) (size 0.8) (drill 0.4) (layers F.Cu B.Cu) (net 8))
 (segment (start 67.056 58.166) (end 70.866 58.166) (width 0.25) (layer F.Cu) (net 8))
 (segment (start 65.571201 59.650799) (end 67.056 58.166) (width 0.25) (layer F.Cu) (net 8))
 (segment (start 69.571201 48.67) (end 69.571201 46.010799) (width 0.25) (layer F.Cu) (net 14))
 (segment (start 69.571201 46.010799) (end 69.862 45.72) (width 0.25) (layer F.Cu) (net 14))
 (segment (start 61.571201 64.67) (end 61.571201 67.413201) (width 0.25) (layer F.Cu) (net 16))
 (segment (start 63.258 69.1) (end 67.31 69.1) (width 0.25) (layer F.Cu) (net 16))
 (segment (start 61.571201 67.413201) (end 63.258 69.1) (width 0.25) (layer F.Cu) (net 16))
 (segment (start 57.571201 64.67) (end 57.571201 62.316799) (width 0.25) (layer F.Cu) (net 17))
 (segment (start 63.571201 62.301201) (end 63.571201 64.67) (width 0.25) (layer F.Cu) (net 17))
 (segment (start 62.738 61.468) (end 63.571201 62.301201) (width 0.25) (layer F.Cu) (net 17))
 (segment (start 58.42 61.468) (end 62.738 61.468) (width 0.25) (layer F.Cu) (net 17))
 (segment (start 57.571201 62.316799) (end 58.42 61.468) (width 0.25) (layer F.Cu) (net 17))
 (segment (start 63.571201 64.67) (end 63.571201 65.349201) (width 0.25) (layer F.Cu) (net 17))
 (segment (start 63.571201 65.349201) (end 65.786 67.564) (width 0.25) (layer F.Cu) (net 17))
 (segment (start 65.786 67.564) (end 69.596 67.564) (width 0.25) (layer F.Cu) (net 17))
 (segment (start 69.596 67.564) (end 70.358 66.802) (width 0.25) (layer F.Cu) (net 17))
 (segment (start 70.358 66.802) (end 72.136 66.802) (width 0.25) (layer F.Cu) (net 17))
 (via (at 72.136 66.802) (size 0.8) (drill 0.4) (layers F.Cu B.Cu) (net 17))
 (segment (start 72.136 66.802) (end 76.962 66.802) (width 0.25) (layer B.Cu) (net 17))
 (via (at 76.962 66.802) (size 0.8) (drill 0.4) (layers F.Cu B.Cu) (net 17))
 (segment (start 76.962 66.802) (end 78.232 66.802) (width 0.25) (layer F.Cu) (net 17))
 (segment (start 78.232 66.802) (end 79.03 66.004) (width 0.25) (layer F.Cu) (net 17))
 (segment (start 79.03 66.004) (end 79.03 63.335) (width 0.25) (layer F.Cu) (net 17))
 (segment (start 79.03 71.285) (end 75.615 71.285) (width 0.25) (layer F.Cu) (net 17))
 (segment (start 75.615 71.285) (end 74.93 70.6) (width 0.25) (layer F.Cu) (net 17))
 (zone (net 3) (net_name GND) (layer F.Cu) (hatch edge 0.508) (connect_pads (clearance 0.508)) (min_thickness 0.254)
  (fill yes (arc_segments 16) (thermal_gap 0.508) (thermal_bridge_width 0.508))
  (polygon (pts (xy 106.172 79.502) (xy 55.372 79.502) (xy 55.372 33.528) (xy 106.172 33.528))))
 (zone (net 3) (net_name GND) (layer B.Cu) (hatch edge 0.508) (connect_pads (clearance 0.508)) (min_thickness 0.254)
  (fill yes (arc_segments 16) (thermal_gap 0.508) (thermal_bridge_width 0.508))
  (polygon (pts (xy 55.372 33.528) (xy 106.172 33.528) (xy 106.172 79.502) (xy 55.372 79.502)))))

